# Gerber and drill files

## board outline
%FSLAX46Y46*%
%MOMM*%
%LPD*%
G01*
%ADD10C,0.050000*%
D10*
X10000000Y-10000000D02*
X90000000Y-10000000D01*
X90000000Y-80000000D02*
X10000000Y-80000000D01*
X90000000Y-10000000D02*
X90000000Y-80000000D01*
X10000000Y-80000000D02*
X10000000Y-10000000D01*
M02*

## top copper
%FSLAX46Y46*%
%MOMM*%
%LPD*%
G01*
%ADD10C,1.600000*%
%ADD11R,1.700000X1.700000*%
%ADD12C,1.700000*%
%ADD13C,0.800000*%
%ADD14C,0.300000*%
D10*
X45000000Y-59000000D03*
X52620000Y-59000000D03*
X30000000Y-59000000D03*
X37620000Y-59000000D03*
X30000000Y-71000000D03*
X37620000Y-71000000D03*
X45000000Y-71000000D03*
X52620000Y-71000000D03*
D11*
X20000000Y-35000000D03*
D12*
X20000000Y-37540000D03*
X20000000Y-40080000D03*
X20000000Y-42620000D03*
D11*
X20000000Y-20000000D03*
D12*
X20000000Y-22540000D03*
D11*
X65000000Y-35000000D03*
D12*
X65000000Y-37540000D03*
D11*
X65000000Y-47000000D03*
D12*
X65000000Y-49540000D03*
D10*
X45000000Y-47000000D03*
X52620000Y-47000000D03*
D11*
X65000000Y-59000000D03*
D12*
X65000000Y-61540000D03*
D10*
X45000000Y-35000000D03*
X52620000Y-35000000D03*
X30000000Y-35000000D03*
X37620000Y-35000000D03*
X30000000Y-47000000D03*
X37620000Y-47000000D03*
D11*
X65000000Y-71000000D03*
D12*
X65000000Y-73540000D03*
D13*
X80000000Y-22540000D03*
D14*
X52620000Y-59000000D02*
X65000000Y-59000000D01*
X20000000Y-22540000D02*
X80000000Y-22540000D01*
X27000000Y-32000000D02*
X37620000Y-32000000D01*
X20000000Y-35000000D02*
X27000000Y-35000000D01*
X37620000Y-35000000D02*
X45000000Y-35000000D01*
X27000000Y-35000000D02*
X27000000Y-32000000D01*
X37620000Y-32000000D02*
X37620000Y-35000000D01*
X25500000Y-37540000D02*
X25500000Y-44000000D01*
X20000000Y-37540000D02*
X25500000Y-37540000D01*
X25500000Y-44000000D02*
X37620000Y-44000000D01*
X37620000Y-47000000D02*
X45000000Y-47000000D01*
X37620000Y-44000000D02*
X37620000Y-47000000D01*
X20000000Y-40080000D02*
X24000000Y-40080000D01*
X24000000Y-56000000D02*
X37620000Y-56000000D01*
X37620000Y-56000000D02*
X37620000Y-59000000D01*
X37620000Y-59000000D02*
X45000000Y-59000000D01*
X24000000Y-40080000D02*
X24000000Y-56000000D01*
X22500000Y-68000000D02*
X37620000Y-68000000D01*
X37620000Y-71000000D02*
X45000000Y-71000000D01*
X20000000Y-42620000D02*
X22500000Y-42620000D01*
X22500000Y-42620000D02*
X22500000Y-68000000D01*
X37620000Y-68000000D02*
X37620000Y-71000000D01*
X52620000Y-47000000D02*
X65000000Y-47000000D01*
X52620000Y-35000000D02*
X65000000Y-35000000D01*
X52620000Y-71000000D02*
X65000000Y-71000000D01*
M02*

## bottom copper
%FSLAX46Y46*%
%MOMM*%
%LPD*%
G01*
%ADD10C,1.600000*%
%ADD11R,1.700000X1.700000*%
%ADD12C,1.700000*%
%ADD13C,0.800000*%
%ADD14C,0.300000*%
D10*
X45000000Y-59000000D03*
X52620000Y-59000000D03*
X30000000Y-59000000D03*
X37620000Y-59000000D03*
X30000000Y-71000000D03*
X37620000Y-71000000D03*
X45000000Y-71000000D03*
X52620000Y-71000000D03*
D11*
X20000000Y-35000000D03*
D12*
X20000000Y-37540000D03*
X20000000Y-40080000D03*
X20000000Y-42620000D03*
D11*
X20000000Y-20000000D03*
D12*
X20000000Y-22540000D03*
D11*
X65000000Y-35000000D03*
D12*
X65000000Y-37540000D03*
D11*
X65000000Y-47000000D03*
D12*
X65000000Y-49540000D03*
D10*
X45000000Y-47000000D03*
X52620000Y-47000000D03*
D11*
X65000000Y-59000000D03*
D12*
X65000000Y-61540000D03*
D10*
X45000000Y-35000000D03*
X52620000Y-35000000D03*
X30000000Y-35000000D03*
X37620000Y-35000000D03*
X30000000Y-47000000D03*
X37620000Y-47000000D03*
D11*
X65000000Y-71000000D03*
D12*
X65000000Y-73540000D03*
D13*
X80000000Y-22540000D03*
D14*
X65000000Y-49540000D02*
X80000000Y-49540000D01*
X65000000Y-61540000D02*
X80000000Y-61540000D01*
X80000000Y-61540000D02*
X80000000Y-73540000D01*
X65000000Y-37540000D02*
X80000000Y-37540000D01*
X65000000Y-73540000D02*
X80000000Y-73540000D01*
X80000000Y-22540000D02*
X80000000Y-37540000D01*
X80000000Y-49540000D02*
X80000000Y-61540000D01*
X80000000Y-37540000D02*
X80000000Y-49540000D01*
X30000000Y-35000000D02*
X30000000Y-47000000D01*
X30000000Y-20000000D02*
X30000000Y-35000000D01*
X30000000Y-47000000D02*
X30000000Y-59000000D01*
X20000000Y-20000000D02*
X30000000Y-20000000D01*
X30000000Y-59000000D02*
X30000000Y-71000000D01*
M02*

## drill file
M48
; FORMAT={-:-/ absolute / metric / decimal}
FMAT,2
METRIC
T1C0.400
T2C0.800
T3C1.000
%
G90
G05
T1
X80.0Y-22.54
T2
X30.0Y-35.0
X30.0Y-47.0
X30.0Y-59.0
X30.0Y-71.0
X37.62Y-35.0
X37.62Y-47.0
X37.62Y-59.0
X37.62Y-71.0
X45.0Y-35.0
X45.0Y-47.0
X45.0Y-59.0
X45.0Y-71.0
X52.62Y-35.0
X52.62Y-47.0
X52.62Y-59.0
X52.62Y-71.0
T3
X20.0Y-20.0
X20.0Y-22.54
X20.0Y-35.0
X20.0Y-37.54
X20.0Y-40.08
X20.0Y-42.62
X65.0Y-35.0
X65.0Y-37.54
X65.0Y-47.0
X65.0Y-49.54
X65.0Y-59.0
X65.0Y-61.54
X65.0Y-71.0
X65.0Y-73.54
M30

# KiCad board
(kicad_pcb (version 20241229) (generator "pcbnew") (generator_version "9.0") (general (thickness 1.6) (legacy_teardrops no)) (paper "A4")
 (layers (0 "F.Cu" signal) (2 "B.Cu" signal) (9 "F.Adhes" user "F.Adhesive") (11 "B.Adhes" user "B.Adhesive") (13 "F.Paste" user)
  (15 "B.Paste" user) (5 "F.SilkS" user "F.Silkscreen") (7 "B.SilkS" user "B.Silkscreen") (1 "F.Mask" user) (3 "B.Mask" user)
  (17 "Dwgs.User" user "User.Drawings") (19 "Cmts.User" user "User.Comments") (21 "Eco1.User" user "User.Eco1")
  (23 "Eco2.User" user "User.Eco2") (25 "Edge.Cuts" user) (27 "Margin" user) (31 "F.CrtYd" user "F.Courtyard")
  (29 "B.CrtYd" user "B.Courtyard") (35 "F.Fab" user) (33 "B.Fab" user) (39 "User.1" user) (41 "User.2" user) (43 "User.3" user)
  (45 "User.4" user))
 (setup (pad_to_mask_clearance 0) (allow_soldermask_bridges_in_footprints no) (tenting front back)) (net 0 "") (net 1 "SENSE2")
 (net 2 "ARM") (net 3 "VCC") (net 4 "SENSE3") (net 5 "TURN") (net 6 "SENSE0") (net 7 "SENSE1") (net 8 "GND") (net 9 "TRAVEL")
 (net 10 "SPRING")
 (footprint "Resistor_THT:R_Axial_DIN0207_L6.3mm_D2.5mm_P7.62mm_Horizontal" (layer "F.Cu") (at 45 59)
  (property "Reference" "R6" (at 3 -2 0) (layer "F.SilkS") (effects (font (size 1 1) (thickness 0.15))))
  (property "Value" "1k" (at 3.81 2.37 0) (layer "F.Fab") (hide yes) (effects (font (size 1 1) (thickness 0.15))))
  (pad "1" thru_hole circle (at 0 0) (size 1.6 1.6) (drill 0.8) (layers "*.Cu" "*.Mask") (remove_unused_layers no) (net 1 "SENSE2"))
  (pad "2" thru_hole circle (at 7.62 0) (size 1.6 1.6) (drill 0.8) (layers "*.Cu" "*.Mask") (remove_unused_layers no) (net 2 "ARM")))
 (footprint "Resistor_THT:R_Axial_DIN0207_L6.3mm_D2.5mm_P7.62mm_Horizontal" (layer "F.Cu") (at 30 59)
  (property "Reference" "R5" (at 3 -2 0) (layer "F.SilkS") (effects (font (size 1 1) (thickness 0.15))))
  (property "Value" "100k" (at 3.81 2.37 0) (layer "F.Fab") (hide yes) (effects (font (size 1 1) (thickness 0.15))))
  (pad "1" thru_hole circle (at 0 0) (size 1.6 1.6) (drill 0.8) (layers "*.Cu" "*.Mask") (remove_unused_layers no) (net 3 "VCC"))
  (pad "2" thru_hole circle (at 7.62 0) (size 1.6 1.6) (drill 0.8) (layers "*.Cu" "*.Mask") (remove_unused_layers no) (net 1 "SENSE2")))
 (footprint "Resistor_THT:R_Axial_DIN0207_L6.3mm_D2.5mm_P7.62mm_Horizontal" (layer "F.Cu") (at 30 71)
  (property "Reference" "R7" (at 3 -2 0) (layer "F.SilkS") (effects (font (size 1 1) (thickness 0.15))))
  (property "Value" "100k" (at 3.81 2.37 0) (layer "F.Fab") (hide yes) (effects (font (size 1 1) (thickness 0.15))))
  (pad "1" thru_hole circle (at 0 0) (size 1.6 1.6) (drill 0.8) (layers "*.Cu" "*.Mask") (remove_unused_layers no) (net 3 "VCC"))
  (pad "2" thru_hole circle (at 7.62 0) (size 1.6 1.6) (drill 0.8) (layers "*.Cu" "*.Mask") (remove_unused_layers no) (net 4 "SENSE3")))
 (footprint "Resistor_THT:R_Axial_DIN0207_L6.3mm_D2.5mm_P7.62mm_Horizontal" (layer "F.Cu") (at 45 71)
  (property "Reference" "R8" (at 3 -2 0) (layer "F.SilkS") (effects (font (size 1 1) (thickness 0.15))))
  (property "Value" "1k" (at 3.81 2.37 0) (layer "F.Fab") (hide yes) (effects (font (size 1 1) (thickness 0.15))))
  (pad "1" thru_hole circle (at 0 0) (size 1.6 1.6) (drill 0.8) (layers "*.Cu" "*.Mask") (remove_unused_layers no) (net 4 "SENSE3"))
  (pad "2" thru_hole circle (at 7.62 0) (size 1.6 1.6) (drill 0.8) (layers "*.Cu" "*.Mask") (remove_unused_layers no) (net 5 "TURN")))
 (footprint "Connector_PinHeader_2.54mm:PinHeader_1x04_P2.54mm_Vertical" (layer "F.Cu") (at 20 35)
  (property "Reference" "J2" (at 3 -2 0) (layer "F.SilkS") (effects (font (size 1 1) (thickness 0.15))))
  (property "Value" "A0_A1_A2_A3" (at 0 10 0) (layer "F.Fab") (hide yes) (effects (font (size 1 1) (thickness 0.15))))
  (pad "1" thru_hole rect (at 0 0) (size 1.7 1.7) (drill 1) (layers "*.Cu" "*.Mask") (remove_unused_layers no) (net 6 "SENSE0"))
  (pad "2" thru_hole circle (at 0 2.54) (size 1.7 1.7) (drill 1) (layers "*.Cu" "*.Mask") (remove_unused_layers no) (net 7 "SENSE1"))
  (pad "3" thru_hole circle (at 0 5.08) (size 1.7 1.7) (drill 1) (layers "*.Cu" "*.Mask") (remove_unused_layers no) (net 1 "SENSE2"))
  (pad "4" thru_hole circle (at 0 7.62) (size 1.7 1.7) (drill 1) (layers "*.Cu" "*.Mask") (remove_unused_layers no) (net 4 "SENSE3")))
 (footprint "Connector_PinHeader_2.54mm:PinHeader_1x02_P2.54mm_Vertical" (layer "F.Cu") (at 20 20)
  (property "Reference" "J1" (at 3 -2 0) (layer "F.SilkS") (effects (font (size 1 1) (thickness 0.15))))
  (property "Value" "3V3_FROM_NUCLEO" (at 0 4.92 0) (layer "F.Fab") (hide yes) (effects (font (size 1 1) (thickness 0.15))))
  (pad "1" thru_hole rect (at 0 0) (size 1.7 1.7) (drill 1) (layers "*.Cu" "*.Mask") (remove_unused_layers no) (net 3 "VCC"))
  (pad "2" thru_hole circle (at 0 2.54) (size 1.7 1.7) (drill 1) (layers "*.Cu" "*.Mask") (remove_unused_layers no) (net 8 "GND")))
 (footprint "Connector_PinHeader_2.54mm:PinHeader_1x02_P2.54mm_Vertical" (layer "F.Cu") (at 65 35)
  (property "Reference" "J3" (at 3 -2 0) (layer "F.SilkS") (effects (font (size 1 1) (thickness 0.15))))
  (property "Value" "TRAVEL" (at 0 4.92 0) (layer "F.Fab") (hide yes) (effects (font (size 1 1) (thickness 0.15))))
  (pad "1" thru_hole rect (at 0 0) (size 1.7 1.7) (drill 1) (layers "*.Cu" "*.Mask") (remove_unused_layers no) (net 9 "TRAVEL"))
  (pad "2" thru_hole circle (at 0 2.54) (size 1.7 1.7) (drill 1) (layers "*.Cu" "*.Mask") (remove_unused_layers no) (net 8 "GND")))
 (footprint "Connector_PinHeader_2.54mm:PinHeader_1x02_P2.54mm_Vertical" (layer "F.Cu") (at 65 47)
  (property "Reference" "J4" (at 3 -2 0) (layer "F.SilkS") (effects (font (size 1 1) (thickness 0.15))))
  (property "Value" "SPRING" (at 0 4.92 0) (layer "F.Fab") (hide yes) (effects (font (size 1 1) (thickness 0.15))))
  (pad "1" thru_hole rect (at 0 0) (size 1.7 1.7) (drill 1) (layers "*.Cu" "*.Mask") (remove_unused_layers no) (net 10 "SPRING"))
  (pad "2" thru_hole circle (at 0 2.54) (size 1.7 1.7) (drill 1) (layers "*.Cu" "*.Mask") (remove_unused_layers no) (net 8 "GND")))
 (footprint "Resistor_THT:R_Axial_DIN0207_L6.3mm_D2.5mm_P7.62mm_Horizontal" (layer "F.Cu") (at 45 47)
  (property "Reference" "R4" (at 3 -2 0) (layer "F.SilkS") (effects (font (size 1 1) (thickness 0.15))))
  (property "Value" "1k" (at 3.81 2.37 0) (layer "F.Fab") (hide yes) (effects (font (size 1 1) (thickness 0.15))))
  (pad "1" thru_hole circle (at 0 0) (size 1.6 1.6) (drill 0.8) (layers "*.Cu" "*.Mask") (remove_unused_layers no) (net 7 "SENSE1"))
  (pad "2" thru_hole circle (at 7.62 0) (size 1.6 1.6) (drill 0.8) (layers "*.Cu" "*.Mask") (remove_unused_layers no) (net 10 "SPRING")))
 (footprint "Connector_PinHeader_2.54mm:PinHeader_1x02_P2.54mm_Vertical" (layer "F.Cu") (at 65 59)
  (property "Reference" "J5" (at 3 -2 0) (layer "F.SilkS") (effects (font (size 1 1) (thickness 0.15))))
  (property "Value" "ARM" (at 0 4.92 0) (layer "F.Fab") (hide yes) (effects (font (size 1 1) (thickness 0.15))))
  (pad "1" thru_hole rect (at 0 0) (size 1.7 1.7) (drill 1) (layers "*.Cu" "*.Mask") (remove_unused_layers no) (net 2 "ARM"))
  (pad "2" thru_hole circle (at 0 2.54) (size 1.7 1.7) (drill 1) (layers "*.Cu" "*.Mask") (remove_unused_layers no) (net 8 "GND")))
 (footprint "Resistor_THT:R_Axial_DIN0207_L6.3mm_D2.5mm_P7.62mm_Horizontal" (layer "F.Cu") (at 45 35)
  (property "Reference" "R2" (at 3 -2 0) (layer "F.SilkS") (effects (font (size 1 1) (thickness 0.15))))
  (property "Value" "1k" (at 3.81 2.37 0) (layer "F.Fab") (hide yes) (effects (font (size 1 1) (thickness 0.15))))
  (pad "1" thru_hole circle (at 0 0) (size 1.6 1.6) (drill 0.8) (layers "*.Cu" "*.Mask") (remove_unused_layers no) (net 6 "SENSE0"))
  (pad "2" thru_hole circle (at 7.62 0) (size 1.6 1.6) (drill 0.8) (layers "*.Cu" "*.Mask") (remove_unused_layers no) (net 9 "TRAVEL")))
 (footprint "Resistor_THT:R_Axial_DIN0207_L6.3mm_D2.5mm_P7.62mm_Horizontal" (layer "F.Cu") (at 30 35)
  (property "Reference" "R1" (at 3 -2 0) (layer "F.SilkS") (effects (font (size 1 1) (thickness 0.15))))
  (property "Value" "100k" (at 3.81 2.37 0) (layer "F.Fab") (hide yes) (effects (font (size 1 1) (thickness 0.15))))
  (pad "1" thru_hole circle (at 0 0) (size 1.6 1.6) (drill 0.8) (layers "*.Cu" "*.Mask") (remove_unused_layers no) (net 3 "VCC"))
  (pad "2" thru_hole circle (at 7.62 0) (size 1.6 1.6) (drill 0.8) (layers "*.Cu" "*.Mask") (remove_unused_layers no) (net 6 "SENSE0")))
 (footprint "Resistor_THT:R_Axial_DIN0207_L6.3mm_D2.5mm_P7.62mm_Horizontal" (layer "F.Cu") (at 30 47)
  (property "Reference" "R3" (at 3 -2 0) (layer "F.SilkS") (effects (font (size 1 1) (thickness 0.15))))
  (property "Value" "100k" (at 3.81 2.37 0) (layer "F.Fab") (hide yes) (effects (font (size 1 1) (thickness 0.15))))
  (pad "1" thru_hole circle (at 0 0) (size 1.6 1.6) (drill 0.8) (layers "*.Cu" "*.Mask") (remove_unused_layers no) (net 3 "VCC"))
  (pad "2" thru_hole circle (at 7.62 0) (size 1.6 1.6) (drill 0.8) (layers "*.Cu" "*.Mask") (remove_unused_layers no) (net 7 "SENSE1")))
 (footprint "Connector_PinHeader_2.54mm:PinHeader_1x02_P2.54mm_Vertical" (layer "F.Cu") (at 65 71)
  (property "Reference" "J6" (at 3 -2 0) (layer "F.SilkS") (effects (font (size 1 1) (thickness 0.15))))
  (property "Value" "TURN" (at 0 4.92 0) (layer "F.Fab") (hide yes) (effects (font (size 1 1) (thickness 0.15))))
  (pad "1" thru_hole rect (at 0 0) (size 1.7 1.7) (drill 1) (layers "*.Cu" "*.Mask") (remove_unused_layers no) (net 5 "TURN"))
  (pad "2" thru_hole circle (at 0 2.54) (size 1.7 1.7) (drill 1) (layers "*.Cu" "*.Mask") (remove_unused_layers no) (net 8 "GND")))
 (gr_line (start 10 10) (end 90 10) (stroke (width 0.05) (type default)) (layer "Edge.Cuts"))
 (gr_line (start 90 80) (end 10 80) (stroke (width 0.05) (type default)) (layer "Edge.Cuts"))
 (gr_line (start 90 10) (end 90 80) (stroke (width 0.05) (type default)) (layer "Edge.Cuts"))
 (gr_line (start 10 80) (end 10 10) (stroke (width 0.05) (type default)) (layer "Edge.Cuts"))
 (segment (start 52.62 59) (end 65 59) (width 0.3) (layer "F.Cu") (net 2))
 (segment (start 20 22.54) (end 80 22.54) (width 0.3) (layer "F.Cu") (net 8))
 (via (at 80 22.54) (size 0.8) (drill 0.4) (layers "F.Cu" "B.Cu") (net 8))
 (segment (start 65 49.54) (end 80 49.54) (width 0.3) (layer "B.Cu") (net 8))
 (segment (start 65 61.54) (end 80 61.54) (width 0.3) (layer "B.Cu") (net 8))
 (segment (start 80 61.54) (end 80 73.54) (width 0.3) (layer "B.Cu") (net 8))
 (segment (start 65 37.54) (end 80 37.54) (width 0.3) (layer "B.Cu") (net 8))
 (segment (start 65 73.54) (end 80 73.54) (width 0.3) (layer "B.Cu") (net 8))
 (segment (start 80 22.54) (end 80 37.54) (width 0.3) (layer "B.Cu") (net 8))
 (segment (start 80 49.54) (end 80 61.54) (width 0.3) (layer "B.Cu") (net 8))
 (segment (start 80 37.54) (end 80 49.54) (width 0.3) (layer "B.Cu") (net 8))
 (segment (start 27 32) (end 37.62 32) (width 0.3) (layer "F.Cu") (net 6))
 (segment (start 20 35) (end 27 35) (width 0.3) (layer "F.Cu") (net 6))
 (segment (start 37.62 35) (end 45 35) (width 0.3) (layer "F.Cu") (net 6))
 (segment (start 27 35) (end 27 32) (width 0.3) (layer "F.Cu") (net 6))
 (segment (start 37.62 32) (end 37.62 35) (width 0.3) (layer "F.Cu") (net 6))
 (segment (start 25.5 37.54) (end 25.5 44) (width 0.3) (layer "F.Cu") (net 7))
 (segment (start 20 37.54) (end 25.5 37.54) (width 0.3) (layer "F.Cu") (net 7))
 (segment (start 25.5 44) (end 37.62 44) (width 0.3) (layer "F.Cu") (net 7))
 (segment (start 37.62 47) (end 45 47) (width 0.3) (layer "F.Cu") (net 7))
 (segment (start 37.62 44) (end 37.62 47) (width 0.3) (layer "F.Cu") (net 7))
 (segment (start 20 40.08) (end 24 40.08) (width 0.3) (layer "F.Cu") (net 1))
 (segment (start 24 56) (end 37.62 56) (width 0.3) (layer "F.Cu") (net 1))
 (segment (start 37.62 56) (end 37.62 59) (width 0.3) (layer "F.Cu") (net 1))
 (segment (start 37.62 59) (end 45 59) (width 0.3) (layer "F.Cu") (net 1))
 (segment (start 24 40.08) (end 24 56) (width 0.3) (layer "F.Cu") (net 1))
 (segment (start 22.5 68) (end 37.62 68) (width 0.3) (layer "F.Cu") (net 4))
 (segment (start 37.62 71) (end 45 71) (width 0.3) (layer "F.Cu") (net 4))
 (segment (start 20 42.62) (end 22.5 42.62) (width 0.3) (layer "F.Cu") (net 4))
 (segment (start 22.5 42.62) (end 22.5 68) (width 0.3) (layer "F.Cu") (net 4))
 (segment (start 37.62 68) (end 37.62 71) (width 0.3) (layer "F.Cu") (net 4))
 (segment (start 52.62 47) (end 65 47) (width 0.3) (layer "F.Cu") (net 10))
 (segment (start 52.62 35) (end 65 35) (width 0.3) (layer "F.Cu") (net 9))
 (segment (start 52.62 71) (end 65 71) (width 0.3) (layer "F.Cu") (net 5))
 (segment (start 30 35) (end 30 47) (width 0.3) (layer "B.Cu") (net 3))
 (segment (start 30 20) (end 30 35) (width 0.3) (layer "B.Cu") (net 3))
 (segment (start 30 47) (end 30 59) (width 0.3) (layer "B.Cu") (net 3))
 (segment (start 20 20) (end 30 20) (width 0.3) (layer "B.Cu") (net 3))
 (segment (start 30 59) (end 30 71) (width 0.3) (layer "B.Cu") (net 3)))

